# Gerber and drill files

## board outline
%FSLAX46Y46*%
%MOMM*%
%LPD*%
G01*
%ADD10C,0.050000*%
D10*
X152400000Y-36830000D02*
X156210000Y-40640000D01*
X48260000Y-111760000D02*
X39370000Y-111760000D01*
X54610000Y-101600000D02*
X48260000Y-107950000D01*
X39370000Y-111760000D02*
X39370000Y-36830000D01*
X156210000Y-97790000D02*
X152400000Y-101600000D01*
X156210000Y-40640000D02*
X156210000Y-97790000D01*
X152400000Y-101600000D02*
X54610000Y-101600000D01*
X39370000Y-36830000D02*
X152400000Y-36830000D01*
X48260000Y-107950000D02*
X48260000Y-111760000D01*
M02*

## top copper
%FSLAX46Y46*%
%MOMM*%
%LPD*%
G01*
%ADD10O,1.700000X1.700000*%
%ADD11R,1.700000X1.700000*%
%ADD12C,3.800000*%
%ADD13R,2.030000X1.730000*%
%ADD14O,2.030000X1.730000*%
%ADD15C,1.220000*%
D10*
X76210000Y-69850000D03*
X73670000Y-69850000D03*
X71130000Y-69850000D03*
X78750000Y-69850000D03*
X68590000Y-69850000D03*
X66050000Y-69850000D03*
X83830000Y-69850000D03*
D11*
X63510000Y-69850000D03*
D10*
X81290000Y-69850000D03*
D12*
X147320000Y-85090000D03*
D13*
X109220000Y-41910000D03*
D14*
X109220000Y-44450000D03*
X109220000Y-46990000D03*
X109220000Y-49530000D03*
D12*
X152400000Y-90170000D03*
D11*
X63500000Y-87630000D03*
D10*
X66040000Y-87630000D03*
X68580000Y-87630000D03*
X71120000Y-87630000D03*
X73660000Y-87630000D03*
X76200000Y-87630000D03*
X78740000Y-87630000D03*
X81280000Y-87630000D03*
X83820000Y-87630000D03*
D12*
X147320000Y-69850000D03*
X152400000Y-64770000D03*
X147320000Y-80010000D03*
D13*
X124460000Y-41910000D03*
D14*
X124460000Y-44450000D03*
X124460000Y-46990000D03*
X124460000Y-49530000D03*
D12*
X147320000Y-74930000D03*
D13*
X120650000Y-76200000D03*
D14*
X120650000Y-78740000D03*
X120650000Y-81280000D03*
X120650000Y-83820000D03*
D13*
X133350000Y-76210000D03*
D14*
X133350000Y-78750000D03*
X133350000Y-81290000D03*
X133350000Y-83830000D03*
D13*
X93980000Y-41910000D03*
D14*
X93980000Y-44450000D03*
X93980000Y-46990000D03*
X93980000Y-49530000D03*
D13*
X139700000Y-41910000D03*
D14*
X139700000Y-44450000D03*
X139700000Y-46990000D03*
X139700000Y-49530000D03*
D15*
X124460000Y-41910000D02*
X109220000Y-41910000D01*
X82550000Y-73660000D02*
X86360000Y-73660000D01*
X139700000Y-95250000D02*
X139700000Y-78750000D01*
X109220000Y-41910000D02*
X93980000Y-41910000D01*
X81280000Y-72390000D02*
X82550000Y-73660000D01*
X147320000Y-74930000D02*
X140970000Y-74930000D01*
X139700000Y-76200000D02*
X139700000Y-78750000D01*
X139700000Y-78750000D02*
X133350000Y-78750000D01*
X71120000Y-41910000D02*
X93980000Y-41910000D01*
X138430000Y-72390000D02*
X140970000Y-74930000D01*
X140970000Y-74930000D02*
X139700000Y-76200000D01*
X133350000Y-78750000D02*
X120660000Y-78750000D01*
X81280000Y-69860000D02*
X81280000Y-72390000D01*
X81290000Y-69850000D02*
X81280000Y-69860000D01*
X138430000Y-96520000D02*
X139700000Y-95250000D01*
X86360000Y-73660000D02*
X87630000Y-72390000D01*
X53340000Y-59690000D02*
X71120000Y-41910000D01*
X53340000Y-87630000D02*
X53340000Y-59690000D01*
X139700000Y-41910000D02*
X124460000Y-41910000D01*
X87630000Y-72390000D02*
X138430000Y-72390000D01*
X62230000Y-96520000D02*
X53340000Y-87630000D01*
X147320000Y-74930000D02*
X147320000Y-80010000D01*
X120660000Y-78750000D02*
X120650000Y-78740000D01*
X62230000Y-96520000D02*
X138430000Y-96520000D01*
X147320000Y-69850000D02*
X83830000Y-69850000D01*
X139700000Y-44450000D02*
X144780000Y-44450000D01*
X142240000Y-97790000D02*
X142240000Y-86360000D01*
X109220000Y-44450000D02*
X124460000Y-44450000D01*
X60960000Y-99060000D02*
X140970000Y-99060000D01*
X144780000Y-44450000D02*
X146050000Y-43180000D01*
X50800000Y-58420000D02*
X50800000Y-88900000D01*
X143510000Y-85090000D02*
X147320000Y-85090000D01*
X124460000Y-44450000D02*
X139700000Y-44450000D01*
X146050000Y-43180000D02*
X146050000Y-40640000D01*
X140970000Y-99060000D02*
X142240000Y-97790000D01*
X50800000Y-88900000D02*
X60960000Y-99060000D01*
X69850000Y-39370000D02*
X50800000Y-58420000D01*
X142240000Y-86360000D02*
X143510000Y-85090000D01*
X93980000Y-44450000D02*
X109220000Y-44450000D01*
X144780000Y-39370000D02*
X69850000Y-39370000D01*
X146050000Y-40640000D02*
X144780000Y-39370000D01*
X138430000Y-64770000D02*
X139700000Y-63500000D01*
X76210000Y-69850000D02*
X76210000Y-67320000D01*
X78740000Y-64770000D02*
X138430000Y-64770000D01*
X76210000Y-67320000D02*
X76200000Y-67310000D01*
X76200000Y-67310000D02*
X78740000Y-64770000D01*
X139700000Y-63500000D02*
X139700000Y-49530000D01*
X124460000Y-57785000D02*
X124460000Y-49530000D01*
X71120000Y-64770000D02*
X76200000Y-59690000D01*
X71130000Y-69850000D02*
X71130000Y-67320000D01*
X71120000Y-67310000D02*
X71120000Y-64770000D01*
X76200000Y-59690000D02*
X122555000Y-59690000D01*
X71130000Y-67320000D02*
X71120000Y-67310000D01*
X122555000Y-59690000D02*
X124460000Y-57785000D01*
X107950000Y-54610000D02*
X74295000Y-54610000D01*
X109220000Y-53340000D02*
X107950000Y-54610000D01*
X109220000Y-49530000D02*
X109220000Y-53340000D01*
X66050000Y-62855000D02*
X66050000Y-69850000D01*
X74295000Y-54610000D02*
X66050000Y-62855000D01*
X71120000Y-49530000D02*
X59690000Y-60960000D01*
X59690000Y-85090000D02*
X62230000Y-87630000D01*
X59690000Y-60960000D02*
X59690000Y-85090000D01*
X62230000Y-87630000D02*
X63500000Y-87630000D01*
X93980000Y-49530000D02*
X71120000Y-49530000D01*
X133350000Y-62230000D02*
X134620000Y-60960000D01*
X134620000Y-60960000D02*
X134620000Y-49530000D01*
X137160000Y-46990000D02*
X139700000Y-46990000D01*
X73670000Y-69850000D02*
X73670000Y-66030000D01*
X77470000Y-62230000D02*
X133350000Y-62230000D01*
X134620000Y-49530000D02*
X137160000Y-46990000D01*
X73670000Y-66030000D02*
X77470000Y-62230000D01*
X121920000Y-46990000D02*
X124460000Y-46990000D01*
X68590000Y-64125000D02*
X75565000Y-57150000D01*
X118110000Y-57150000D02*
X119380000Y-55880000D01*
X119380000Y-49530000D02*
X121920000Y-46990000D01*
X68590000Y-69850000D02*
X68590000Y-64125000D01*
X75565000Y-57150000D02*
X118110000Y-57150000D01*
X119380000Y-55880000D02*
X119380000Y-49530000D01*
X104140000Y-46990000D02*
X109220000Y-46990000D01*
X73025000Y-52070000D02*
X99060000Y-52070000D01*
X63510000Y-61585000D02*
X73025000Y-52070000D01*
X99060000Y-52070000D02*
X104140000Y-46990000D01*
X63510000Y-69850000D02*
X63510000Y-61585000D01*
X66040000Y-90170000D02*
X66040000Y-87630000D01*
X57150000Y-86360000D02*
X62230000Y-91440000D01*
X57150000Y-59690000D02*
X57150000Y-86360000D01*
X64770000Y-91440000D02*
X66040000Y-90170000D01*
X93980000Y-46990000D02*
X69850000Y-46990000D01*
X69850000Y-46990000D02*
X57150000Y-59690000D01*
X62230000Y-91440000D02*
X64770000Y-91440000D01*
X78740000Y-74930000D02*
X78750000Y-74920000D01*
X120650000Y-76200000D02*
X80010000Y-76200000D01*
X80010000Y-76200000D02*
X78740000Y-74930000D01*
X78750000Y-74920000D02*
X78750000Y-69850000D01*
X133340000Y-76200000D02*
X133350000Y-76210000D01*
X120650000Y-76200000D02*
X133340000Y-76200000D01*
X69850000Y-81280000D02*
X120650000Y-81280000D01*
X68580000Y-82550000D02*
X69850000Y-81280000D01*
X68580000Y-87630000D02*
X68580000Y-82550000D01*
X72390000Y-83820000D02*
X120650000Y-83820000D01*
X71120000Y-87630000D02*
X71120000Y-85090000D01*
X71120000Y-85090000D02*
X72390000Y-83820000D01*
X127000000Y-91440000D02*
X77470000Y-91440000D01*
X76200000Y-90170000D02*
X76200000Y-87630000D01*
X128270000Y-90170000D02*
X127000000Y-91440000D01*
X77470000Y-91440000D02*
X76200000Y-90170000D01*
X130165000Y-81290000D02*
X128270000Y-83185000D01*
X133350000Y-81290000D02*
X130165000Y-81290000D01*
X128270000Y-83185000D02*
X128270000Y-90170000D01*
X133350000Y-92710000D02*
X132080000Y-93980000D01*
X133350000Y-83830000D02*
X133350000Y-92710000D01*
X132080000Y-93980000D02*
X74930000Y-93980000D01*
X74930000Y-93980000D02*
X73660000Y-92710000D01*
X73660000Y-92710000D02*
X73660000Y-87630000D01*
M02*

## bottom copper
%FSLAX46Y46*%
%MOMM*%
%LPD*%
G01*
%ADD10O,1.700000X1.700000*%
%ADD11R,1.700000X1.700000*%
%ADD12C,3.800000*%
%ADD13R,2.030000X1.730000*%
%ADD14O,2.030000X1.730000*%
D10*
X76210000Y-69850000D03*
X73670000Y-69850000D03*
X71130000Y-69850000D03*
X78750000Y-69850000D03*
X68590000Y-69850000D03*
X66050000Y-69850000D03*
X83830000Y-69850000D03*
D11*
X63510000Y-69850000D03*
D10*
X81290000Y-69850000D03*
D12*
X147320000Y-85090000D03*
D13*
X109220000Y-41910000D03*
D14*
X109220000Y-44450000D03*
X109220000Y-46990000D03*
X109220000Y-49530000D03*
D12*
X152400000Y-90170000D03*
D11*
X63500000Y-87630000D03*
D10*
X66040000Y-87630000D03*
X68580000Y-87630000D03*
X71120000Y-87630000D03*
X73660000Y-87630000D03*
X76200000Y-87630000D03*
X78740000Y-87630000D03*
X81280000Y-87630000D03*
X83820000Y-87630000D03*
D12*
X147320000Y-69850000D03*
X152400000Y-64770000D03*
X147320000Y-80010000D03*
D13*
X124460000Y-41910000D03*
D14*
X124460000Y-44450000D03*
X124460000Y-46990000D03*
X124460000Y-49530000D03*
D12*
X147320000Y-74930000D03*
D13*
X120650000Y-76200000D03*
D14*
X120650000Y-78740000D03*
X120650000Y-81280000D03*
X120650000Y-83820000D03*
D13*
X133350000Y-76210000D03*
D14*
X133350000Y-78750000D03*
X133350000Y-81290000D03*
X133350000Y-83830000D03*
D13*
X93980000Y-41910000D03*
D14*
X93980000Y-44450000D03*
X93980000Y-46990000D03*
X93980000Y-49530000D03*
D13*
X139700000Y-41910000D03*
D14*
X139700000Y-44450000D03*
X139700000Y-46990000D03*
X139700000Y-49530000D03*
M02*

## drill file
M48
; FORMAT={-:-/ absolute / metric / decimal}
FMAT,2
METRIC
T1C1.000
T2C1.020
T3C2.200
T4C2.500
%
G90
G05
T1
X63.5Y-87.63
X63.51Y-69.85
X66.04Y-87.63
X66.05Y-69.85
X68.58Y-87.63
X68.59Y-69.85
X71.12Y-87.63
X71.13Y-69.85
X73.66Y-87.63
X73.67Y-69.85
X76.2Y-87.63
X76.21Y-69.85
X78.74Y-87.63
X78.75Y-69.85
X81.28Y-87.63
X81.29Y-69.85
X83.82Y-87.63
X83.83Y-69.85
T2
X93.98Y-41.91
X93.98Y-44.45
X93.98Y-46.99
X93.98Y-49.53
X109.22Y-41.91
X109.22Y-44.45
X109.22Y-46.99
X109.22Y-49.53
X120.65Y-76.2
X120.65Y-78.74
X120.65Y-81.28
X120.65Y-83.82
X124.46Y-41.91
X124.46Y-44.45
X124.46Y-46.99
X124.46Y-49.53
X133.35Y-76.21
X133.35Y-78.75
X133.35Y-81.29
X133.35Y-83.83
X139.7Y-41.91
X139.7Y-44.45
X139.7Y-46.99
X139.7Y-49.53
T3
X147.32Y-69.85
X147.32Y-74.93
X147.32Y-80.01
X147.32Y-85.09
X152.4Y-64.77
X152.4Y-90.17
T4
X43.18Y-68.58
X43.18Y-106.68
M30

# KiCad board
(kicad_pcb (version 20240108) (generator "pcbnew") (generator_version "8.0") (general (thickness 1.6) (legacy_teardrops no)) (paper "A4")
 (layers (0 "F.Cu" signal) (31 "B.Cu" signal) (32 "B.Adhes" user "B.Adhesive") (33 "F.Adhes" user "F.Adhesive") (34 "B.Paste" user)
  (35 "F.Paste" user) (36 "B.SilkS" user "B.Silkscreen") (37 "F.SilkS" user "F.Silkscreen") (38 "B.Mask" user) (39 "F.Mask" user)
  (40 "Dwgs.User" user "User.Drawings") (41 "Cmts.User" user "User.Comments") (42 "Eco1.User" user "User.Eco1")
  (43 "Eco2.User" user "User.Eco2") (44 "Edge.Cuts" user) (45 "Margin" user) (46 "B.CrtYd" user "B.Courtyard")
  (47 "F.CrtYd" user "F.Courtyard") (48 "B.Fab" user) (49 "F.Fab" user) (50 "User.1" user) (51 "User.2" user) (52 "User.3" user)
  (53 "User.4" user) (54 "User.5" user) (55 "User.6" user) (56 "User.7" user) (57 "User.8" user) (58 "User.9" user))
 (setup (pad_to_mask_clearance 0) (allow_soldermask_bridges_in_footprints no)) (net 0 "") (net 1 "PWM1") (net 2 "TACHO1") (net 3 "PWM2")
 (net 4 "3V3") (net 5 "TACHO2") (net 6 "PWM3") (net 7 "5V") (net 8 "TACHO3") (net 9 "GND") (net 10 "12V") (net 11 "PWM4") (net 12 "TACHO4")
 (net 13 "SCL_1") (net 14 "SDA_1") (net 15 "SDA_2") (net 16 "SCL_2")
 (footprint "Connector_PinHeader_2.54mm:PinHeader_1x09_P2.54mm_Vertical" (layer "F.Cu") (at 63.51 69.85 90)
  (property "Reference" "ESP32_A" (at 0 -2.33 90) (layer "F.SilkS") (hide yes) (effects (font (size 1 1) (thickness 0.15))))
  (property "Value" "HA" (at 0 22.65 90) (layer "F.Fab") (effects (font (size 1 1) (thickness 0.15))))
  (pad "1" thru_hole oval (at 0 12.7 90) (size 1.7 1.7) (drill 1) (layers "*.Cu" "*.Mask") (remove_unused_layers no) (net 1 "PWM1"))
  (pad "2" thru_hole oval (at 0 10.16 90) (size 1.7 1.7) (drill 1) (layers "*.Cu" "*.Mask") (remove_unused_layers no) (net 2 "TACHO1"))
  (pad "3" thru_hole oval (at 0 7.62 90) (size 1.7 1.7) (drill 1) (layers "*.Cu" "*.Mask") (remove_unused_layers no) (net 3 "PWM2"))
  (pad "3V3" thru_hole oval (at 0 15.24 90) (size 1.7 1.7) (drill 1) (layers "*.Cu" "*.Mask") (remove_unused_layers no) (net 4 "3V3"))
  (pad "4" thru_hole oval (at 0 5.08 90) (size 1.7 1.7) (drill 1) (layers "*.Cu" "*.Mask") (remove_unused_layers no) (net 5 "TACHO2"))
  (pad "5" thru_hole oval (at 0 2.54 90) (size 1.7 1.7) (drill 1) (layers "*.Cu" "*.Mask") (remove_unused_layers no) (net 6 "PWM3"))
  (pad "5V" thru_hole oval (at 0 20.32 90) (size 1.7 1.7) (drill 1) (layers "*.Cu" "*.Mask") (remove_unused_layers no) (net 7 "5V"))
  (pad "6" thru_hole rect (at 0 0 90) (size 1.7 1.7) (drill 1) (layers "*.Cu" "*.Mask") (remove_unused_layers no) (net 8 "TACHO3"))
  (pad "GND" thru_hole oval (at 0 17.78 90) (size 1.7 1.7) (drill 1) (layers "*.Cu" "*.Mask") (remove_unused_layers no) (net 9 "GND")))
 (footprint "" (layer "F.Cu") (at 147.32 85.09)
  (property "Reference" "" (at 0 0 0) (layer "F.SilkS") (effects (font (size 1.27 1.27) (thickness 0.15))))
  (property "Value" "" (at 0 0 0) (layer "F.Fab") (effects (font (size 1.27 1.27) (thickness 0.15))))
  (pad "1" thru_hole circle (at 0 0) (size 3.8 3.8) (drill 2.2) (layers "*.Cu" "*.Mask") (remove_unused_layers no) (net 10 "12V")))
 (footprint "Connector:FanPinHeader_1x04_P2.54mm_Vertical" (layer "F.Cu") (at 109.22 41.91 -90)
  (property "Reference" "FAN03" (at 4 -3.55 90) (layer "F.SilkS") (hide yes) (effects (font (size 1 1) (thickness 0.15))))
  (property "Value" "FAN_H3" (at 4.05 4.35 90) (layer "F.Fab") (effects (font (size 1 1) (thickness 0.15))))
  (pad "1" thru_hole rect (at 0 0) (size 2.03 1.73) (drill 1.02) (layers "*.Cu" "*.Mask") (remove_unused_layers no) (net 9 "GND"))
  (pad "2" thru_hole oval (at 2.54 0) (size 2.03 1.73) (drill 1.02) (layers "*.Cu" "*.Mask") (remove_unused_layers no) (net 10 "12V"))
  (pad "3" thru_hole oval (at 5.08 0) (size 2.03 1.73) (drill 1.02) (layers "*.Cu" "*.Mask") (remove_unused_layers no) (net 8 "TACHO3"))
  (pad "4" thru_hole oval (at 7.62 0) (size 2.03 1.73) (drill 1.02) (layers "*.Cu" "*.Mask") (remove_unused_layers no) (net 6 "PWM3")))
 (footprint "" (layer "F.Cu") (at 152.4 90.17)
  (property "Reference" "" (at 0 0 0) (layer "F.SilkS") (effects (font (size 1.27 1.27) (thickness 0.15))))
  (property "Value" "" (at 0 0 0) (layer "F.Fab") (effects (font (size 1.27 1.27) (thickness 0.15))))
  (pad "MNT" thru_hole circle (at 0 0) (size 3.8 3.8) (drill 2.2) (layers "*.Cu" "*.Mask") (remove_unused_layers no)))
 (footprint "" (layer "F.Cu") (at 43.18 106.68)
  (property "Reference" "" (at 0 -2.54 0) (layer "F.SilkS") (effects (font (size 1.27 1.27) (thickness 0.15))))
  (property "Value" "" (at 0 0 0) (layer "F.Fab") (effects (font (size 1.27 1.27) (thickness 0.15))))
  (pad "" np_thru_hole circle (at 0 0) (size 2.5 2.5) (drill 2.5) (layers "*.Cu" "*.Mask")))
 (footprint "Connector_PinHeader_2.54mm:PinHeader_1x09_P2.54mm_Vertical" (layer "F.Cu") (at 63.5 87.63 90)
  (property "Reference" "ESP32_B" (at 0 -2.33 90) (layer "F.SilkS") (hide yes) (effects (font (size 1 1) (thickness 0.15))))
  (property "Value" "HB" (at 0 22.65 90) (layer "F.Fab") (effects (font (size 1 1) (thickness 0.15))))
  (pad "7" thru_hole rect (at 0 0 90) (size 1.7 1.7) (drill 1) (layers "*.Cu" "*.Mask") (remove_unused_layers no) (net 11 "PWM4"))
  (pad "8" thru_hole oval (at 0 2.54 90) (size 1.7 1.7) (drill 1) (layers "*.Cu" "*.Mask") (remove_unused_layers no) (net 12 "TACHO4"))
  (pad "9" thru_hole oval (at 0 5.08 90) (size 1.7 1.7) (drill 1) (layers "*.Cu" "*.Mask") (remove_unused_layers no) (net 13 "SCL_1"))
  (pad "10" thru_hole oval (at 0 7.62 90) (size 1.7 1.7) (drill 1) (layers "*.Cu" "*.Mask") (remove_unused_layers no) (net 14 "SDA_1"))
  (pad "11" thru_hole oval (at 0 10.16 90) (size 1.7 1.7) (drill 1) (layers "*.Cu" "*.Mask") (remove_unused_layers no) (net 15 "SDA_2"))
  (pad "12" thru_hole oval (at 0 12.7 90) (size 1.7 1.7) (drill 1) (layers "*.Cu" "*.Mask") (remove_unused_layers no) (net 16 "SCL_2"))
  (pad "13" thru_hole oval (at 0 15.24 90) (size 1.7 1.7) (drill 1) (layers "*.Cu" "*.Mask") (remove_unused_layers no))
  (pad "RX" thru_hole oval (at 0 17.78 90) (size 1.7 1.7) (drill 1) (layers "*.Cu" "*.Mask") (remove_unused_layers no))
  (pad "TX" thru_hole oval (at 0 20.32 90) (size 1.7 1.7) (drill 1) (layers "*.Cu" "*.Mask") (remove_unused_layers no)))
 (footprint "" (layer "F.Cu") (at 147.32 69.85)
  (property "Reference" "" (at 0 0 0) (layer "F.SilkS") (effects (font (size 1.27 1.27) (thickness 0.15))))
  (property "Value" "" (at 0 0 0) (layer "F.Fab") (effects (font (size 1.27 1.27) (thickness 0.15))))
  (pad "4" thru_hole circle (at 0 0) (size 3.8 3.8) (drill 2.2) (layers "*.Cu" "*.Mask") (remove_unused_layers no) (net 7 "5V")))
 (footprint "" (layer "F.Cu") (at 152.4 64.77)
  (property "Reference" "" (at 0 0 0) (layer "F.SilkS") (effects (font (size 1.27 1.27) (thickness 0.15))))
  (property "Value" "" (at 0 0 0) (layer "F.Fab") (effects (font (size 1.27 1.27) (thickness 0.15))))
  (pad "MNT" thru_hole circle (at 0 0) (size 3.8 3.8) (drill 2.2) (layers "*.Cu" "*.Mask") (remove_unused_layers no)))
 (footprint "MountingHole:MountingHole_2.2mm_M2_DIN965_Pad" (layer "F.Cu") (at 147.32 80.01)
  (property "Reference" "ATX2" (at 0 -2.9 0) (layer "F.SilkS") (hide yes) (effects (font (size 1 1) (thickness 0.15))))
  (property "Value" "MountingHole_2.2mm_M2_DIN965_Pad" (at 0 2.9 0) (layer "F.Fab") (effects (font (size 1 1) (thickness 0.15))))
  (pad "2" thru_hole circle (at 0 0) (size 3.8 3.8) (drill 2.2) (layers "*.Cu" "*.Mask") (remove_unused_layers no) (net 9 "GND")))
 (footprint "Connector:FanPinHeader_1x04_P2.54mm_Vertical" (layer "F.Cu") (at 124.46 41.91 -90)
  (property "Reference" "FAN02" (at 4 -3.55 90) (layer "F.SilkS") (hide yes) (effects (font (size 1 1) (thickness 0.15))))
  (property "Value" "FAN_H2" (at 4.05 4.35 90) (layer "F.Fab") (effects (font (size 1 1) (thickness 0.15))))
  (pad "1" thru_hole rect (at 0 0) (size 2.03 1.73) (drill 1.02) (layers "*.Cu" "*.Mask") (remove_unused_layers no) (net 9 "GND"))
  (pad "2" thru_hole oval (at 2.54 0) (size 2.03 1.73) (drill 1.02) (layers "*.Cu" "*.Mask") (remove_unused_layers no) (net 10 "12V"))
  (pad "3" thru_hole oval (at 5.08 0) (size 2.03 1.73) (drill 1.02) (layers "*.Cu" "*.Mask") (remove_unused_layers no) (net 5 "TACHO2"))
  (pad "4" thru_hole oval (at 7.62 0) (size 2.03 1.73) (drill 1.02) (layers "*.Cu" "*.Mask") (remove_unused_layers no) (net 3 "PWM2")))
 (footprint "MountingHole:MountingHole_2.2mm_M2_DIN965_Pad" (layer "F.Cu") (at 147.32 74.93)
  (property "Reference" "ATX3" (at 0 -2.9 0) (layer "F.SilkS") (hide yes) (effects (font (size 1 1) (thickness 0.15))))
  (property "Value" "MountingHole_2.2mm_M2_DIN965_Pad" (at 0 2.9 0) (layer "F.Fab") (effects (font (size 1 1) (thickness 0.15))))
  (pad "3" thru_hole circle (at 0 0) (size 3.8 3.8) (drill 2.2) (layers "*.Cu" "*.Mask") (remove_unused_layers no) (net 9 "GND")))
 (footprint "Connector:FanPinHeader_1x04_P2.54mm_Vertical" (layer "F.Cu") (at 120.65 76.2 -90)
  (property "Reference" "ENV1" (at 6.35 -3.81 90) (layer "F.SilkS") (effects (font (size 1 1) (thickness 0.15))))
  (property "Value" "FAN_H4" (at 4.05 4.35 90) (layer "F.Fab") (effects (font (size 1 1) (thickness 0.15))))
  (pad "1" thru_hole rect (at 0 0) (size 2.03 1.73) (drill 1.02) (layers "*.Cu" "*.Mask") (remove_unused_layers no) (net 4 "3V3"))
  (pad "2" thru_hole oval (at 2.54 0) (size 2.03 1.73) (drill 1.02) (layers "*.Cu" "*.Mask") (remove_unused_layers no) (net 9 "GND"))
  (pad "3" thru_hole oval (at 5.08 0) (size 2.03 1.73) (drill 1.02) (layers "*.Cu" "*.Mask") (remove_unused_layers no) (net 13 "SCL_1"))
  (pad "4" thru_hole oval (at 7.62 0) (size 2.03 1.73) (drill 1.02) (layers "*.Cu" "*.Mask") (remove_unused_layers no) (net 14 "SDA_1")))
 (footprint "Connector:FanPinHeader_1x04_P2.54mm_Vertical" (layer "F.Cu") (at 133.35 76.21 -90)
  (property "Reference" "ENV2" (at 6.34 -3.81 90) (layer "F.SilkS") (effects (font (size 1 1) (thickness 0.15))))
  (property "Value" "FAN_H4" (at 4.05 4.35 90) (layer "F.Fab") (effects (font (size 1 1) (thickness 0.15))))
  (pad "1" thru_hole rect (at 0 0) (size 2.03 1.73) (drill 1.02) (layers "*.Cu" "*.Mask") (remove_unused_layers no) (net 4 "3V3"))
  (pad "2" thru_hole oval (at 2.54 0) (size 2.03 1.73) (drill 1.02) (layers "*.Cu" "*.Mask") (remove_unused_layers no) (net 9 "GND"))
  (pad "3" thru_hole oval (at 5.08 0) (size 2.03 1.73) (drill 1.02) (layers "*.Cu" "*.Mask") (remove_unused_layers no) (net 16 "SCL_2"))
  (pad "4" thru_hole oval (at 7.62 0) (size 2.03 1.73) (drill 1.02) (layers "*.Cu" "*.Mask") (remove_unused_layers no) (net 15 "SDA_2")))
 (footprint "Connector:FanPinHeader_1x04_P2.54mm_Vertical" (layer "F.Cu") (at 93.98 41.91 -90)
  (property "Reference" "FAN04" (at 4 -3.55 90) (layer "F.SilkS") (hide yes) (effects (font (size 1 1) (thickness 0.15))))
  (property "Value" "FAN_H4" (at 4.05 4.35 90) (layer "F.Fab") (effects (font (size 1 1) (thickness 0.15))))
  (pad "1" thru_hole rect (at 0 0) (size 2.03 1.73) (drill 1.02) (layers "*.Cu" "*.Mask") (remove_unused_layers no) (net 9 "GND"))
  (pad "2" thru_hole oval (at 2.54 0) (size 2.03 1.73) (drill 1.02) (layers "*.Cu" "*.Mask") (remove_unused_layers no) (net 10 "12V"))
  (pad "3" thru_hole oval (at 5.08 0) (size 2.03 1.73) (drill 1.02) (layers "*.Cu" "*.Mask") (remove_unused_layers no) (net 12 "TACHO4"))
  (pad "4" thru_hole oval (at 7.62 0) (size 2.03 1.73) (drill 1.02) (layers "*.Cu" "*.Mask") (remove_unused_layers no) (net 11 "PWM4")))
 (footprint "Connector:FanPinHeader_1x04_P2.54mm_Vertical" (layer "F.Cu") (at 139.7 41.91 -90)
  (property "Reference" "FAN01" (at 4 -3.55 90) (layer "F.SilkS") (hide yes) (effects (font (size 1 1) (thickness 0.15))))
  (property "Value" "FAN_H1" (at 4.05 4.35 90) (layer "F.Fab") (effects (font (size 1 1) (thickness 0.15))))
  (pad "1" thru_hole rect (at 0 0) (size 2.03 1.73) (drill 1.02) (layers "*.Cu" "*.Mask") (remove_unused_layers no) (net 9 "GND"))
  (pad "2" thru_hole oval (at 2.54 0) (size 2.03 1.73) (drill 1.02) (layers "*.Cu" "*.Mask") (remove_unused_layers no) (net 10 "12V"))
  (pad "3" thru_hole oval (at 5.08 0) (size 2.03 1.73) (drill 1.02) (layers "*.Cu" "*.Mask") (remove_unused_layers no) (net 2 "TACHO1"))
  (pad "4" thru_hole oval (at 7.62 0) (size 2.03 1.73) (drill 1.02) (layers "*.Cu" "*.Mask") (remove_unused_layers no) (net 1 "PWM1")))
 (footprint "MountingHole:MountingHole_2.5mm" (layer "F.Cu") (at 43.18 68.58)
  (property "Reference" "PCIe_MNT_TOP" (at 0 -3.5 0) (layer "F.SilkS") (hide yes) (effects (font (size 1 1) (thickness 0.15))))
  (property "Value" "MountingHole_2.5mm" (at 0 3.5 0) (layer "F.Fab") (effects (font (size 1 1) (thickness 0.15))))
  (pad "" np_thru_hole circle (at 0 0) (size 2.5 2.5) (drill 2.5) (layers "*.Cu" "*.Mask")))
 (gr_line (start 152.4 36.83) (end 156.21 40.64) (stroke (width 0.05) (type default)) (layer "Edge.Cuts"))
 (gr_line (start 48.26 111.76) (end 39.37 111.76) (stroke (width 0.05) (type default)) (layer "Edge.Cuts"))
 (gr_line (start 54.61 101.6) (end 48.26 107.95) (stroke (width 0.05) (type default)) (layer "Edge.Cuts"))
 (gr_line (start 39.37 111.76) (end 39.37 36.83) (stroke (width 0.05) (type default)) (layer "Edge.Cuts"))
 (gr_line (start 156.21 97.79) (end 152.4 101.6) (stroke (width 0.05) (type default)) (layer "Edge.Cuts"))
 (gr_line (start 156.21 40.64) (end 156.21 97.79) (stroke (width 0.05) (type default)) (layer "Edge.Cuts"))
 (gr_line (start 152.4 101.6) (end 54.61 101.6) (stroke (width 0.05) (type default)) (layer "Edge.Cuts"))
 (gr_line (start 39.37 36.83) (end 152.4 36.83) (stroke (width 0.05) (type default)) (layer "Edge.Cuts"))
 (gr_line (start 48.26 107.95) (end 48.26 111.76) (stroke (width 0.05) (type default)) (layer "Edge.Cuts"))
 (segment (start 124.46 41.91) (end 109.22 41.91) (width 1.22) (layer "F.Cu") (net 9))
 (segment (start 82.55 73.66) (end 86.36 73.66) (width 1.22) (layer "F.Cu") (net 9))
 (segment (start 139.7 95.25) (end 139.7 78.75) (width 1.22) (layer "F.Cu") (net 9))
 (segment (start 109.22 41.91) (end 93.98 41.91) (width 1.22) (layer "F.Cu") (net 9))
 (segment (start 81.28 72.39) (end 82.55 73.66) (width 1.22) (layer "F.Cu") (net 9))
 (segment (start 147.32 74.93) (end 140.97 74.93) (width 1.22) (layer "F.Cu") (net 9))
 (segment (start 139.7 76.2) (end 139.7 78.75) (width 1.22) (layer "F.Cu") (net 9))
 (segment (start 139.7 78.75) (end 133.35 78.75) (width 1.22) (layer "F.Cu") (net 9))
 (segment (start 71.12 41.91) (end 93.98 41.91) (width 1.22) (layer "F.Cu") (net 9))
 (segment (start 138.43 72.39) (end 140.97 74.93) (width 1.22) (layer "F.Cu") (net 9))
 (segment (start 140.97 74.93) (end 139.7 76.2) (width 1.22) (layer "F.Cu") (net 9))
 (segment (start 133.35 78.75) (end 120.66 78.75) (width 1.22) (layer "F.Cu") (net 9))
 (segment (start 81.28 69.86) (end 81.28 72.39) (width 1.22) (layer "F.Cu") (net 9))
 (segment (start 81.29 69.85) (end 81.28 69.86) (width 1.22) (layer "F.Cu") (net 9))
 (segment (start 138.43 96.52) (end 139.7 95.25) (width 1.22) (layer "F.Cu") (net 9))
 (segment (start 86.36 73.66) (end 87.63 72.39) (width 1.22) (layer "F.Cu") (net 9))
 (segment (start 53.34 59.69) (end 71.12 41.91) (width 1.22) (layer "F.Cu") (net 9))
 (segment (start 53.34 87.63) (end 53.34 59.69) (width 1.22) (layer "F.Cu") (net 9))
 (segment (start 139.7 41.91) (end 124.46 41.91) (width 1.22) (layer "F.Cu") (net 9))
 (segment (start 87.63 72.39) (end 138.43 72.39) (width 1.22) (layer "F.Cu") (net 9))
 (segment (start 62.23 96.52) (end 53.34 87.63) (width 1.22) (layer "F.Cu") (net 9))
 (segment (start 147.32 74.93) (end 147.32 80.01) (width 1.22) (layer "F.Cu") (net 9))
 (segment (start 120.66 78.75) (end 120.65 78.74) (width 1.22) (layer "F.Cu") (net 9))
 (segment (start 62.23 96.52) (end 138.43 96.52) (width 1.22) (layer "F.Cu") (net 9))
 (segment (start 147.32 69.85) (end 83.83 69.85) (width 1.22) (layer "F.Cu") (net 7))
 (segment (start 139.7 44.45) (end 144.78 44.45) (width 1.22) (layer "F.Cu") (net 10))
 (segment (start 142.24 97.79) (end 142.24 86.36) (width 1.22) (layer "F.Cu") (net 10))
 (segment (start 109.22 44.45) (end 124.46 44.45) (width 1.22) (layer "F.Cu") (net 10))
 (segment (start 60.96 99.06) (end 140.97 99.06) (width 1.22) (layer "F.Cu") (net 10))
 (segment (start 144.78 44.45) (end 146.05 43.18) (width 1.22) (layer "F.Cu") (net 10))
 (segment (start 50.8 58.42) (end 50.8 88.9) (width 1.22) (layer "F.Cu") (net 10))
 (segment (start 143.51 85.09) (end 147.32 85.09) (width 1.22) (layer "F.Cu") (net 10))
 (segment (start 124.46 44.45) (end 139.7 44.45) (width 1.22) (layer "F.Cu") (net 10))
 (segment (start 146.05 43.18) (end 146.05 40.64) (width 1.22) (layer "F.Cu") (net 10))
 (segment (start 140.97 99.06) (end 142.24 97.79) (width 1.22) (layer "F.Cu") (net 10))
 (segment (start 50.8 88.9) (end 60.96 99.06) (width 1.22) (layer "F.Cu") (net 10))
 (segment (start 69.85 39.37) (end 50.8 58.42) (width 1.22) (layer "F.Cu") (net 10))
 (segment (start 142.24 86.36) (end 143.51 85.09) (width 1.22) (layer "F.Cu") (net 10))
 (segment (start 93.98 44.45) (end 109.22 44.45) (width 1.22) (layer "F.Cu") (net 10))
 (segment (start 144.78 39.37) (end 69.85 39.37) (width 1.22) (layer "F.Cu") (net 10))
 (segment (start 146.05 40.64) (end 144.78 39.37) (width 1.22) (layer "F.Cu") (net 10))
 (segment (start 138.43 64.77) (end 139.7 63.5) (width 1.22) (layer "F.Cu") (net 1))
 (segment (start 76.21 69.85) (end 76.21 67.32) (width 1.22) (layer "F.Cu") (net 1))
 (segment (start 78.74 64.77) (end 138.43 64.77) (width 1.22) (layer "F.Cu") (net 1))
 (segment (start 76.21 67.32) (end 76.2 67.31) (width 1.22) (layer "F.Cu") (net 1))
 (segment (start 76.2 67.31) (end 78.74 64.77) (width 1.22) (layer "F.Cu") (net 1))
 (segment (start 139.7 63.5) (end 139.7 49.53) (width 1.22) (layer "F.Cu") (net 1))
 (segment (start 124.46 57.785) (end 124.46 49.53) (width 1.22) (layer "F.Cu") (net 3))
 (segment (start 71.12 64.77) (end 76.2 59.69) (width 1.22) (layer "F.Cu") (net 3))
 (segment (start 71.13 69.85) (end 71.13 67.32) (width 1.22) (layer "F.Cu") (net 3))
 (segment (start 71.12 67.31) (end 71.12 64.77) (width 1.22) (layer "F.Cu") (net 3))
 (segment (start 76.2 59.69) (end 122.555 59.69) (width 1.22) (layer "F.Cu") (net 3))
 (segment (start 71.13 67.32) (end 71.12 67.31) (width 1.22) (layer "F.Cu") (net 3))
 (segment (start 122.555 59.69) (end 124.46 57.785) (width 1.22) (layer "F.Cu") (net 3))
 (segment (start 107.95 54.61) (end 74.295 54.61) (width 1.22) (layer "F.Cu") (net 6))
 (segment (start 109.22 53.34) (end 107.95 54.61) (width 1.22) (layer "F.Cu") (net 6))
 (segment (start 109.22 49.53) (end 109.22 53.34) (width 1.22) (layer "F.Cu") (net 6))
 (segment (start 66.05 62.855) (end 66.05 69.85) (width 1.22) (layer "F.Cu") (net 6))
 (segment (start 74.295 54.61) (end 66.05 62.855) (width 1.22) (layer "F.Cu") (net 6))
 (segment (start 71.12 49.53) (end 59.69 60.96) (width 1.22) (layer "F.Cu") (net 11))
 (segment (start 59.69 85.09) (end 62.23 87.63) (width 1.22) (layer "F.Cu") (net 11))
 (segment (start 59.69 60.96) (end 59.69 85.09) (width 1.22) (layer "F.Cu") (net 11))
 (segment (start 62.23 87.63) (end 63.5 87.63) (width 1.22) (layer "F.Cu") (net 11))
 (segment (start 93.98 49.53) (end 71.12 49.53) (width 1.22) (layer "F.Cu") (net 11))
 (segment (start 133.35 62.23) (end 134.62 60.96) (width 1.22) (layer "F.Cu") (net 2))
 (segment (start 134.62 60.96) (end 134.62 49.53) (width 1.22) (layer "F.Cu") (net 2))
 (segment (start 137.16 46.99) (end 139.7 46.99) (width 1.22) (layer "F.Cu") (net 2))
 (segment (start 73.67 69.85) (end 73.67 66.03) (width 1.22) (layer "F.Cu") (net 2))
 (segment (start 77.47 62.23) (end 133.35 62.23) (width 1.22) (layer "F.Cu") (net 2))
 (segment (start 134.62 49.53) (end 137.16 46.99) (width 1.22) (layer "F.Cu") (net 2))
 (segment (start 73.67 66.03) (end 77.47 62.23) (width 1.22) (layer "F.Cu") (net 2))
 (segment (start 121.92 46.99) (end 124.46 46.99) (width 1.22) (layer "F.Cu") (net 5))
 (segment (start 68.59 64.125) (end 75.565 57.15) (width 1.22) (layer "F.Cu") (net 5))
 (segment (start 118.11 57.15) (end 119.38 55.88) (width 1.22) (layer "F.Cu") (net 5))
 (segment (start 119.38 49.53) (end 121.92 46.99) (width 1.22) (layer "F.Cu") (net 5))
 (segment (start 68.59 69.85) (end 68.59 64.125) (width 1.22) (layer "F.Cu") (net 5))
 (segment (start 75.565 57.15) (end 118.11 57.15) (width 1.22) (layer "F.Cu") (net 5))
 (segment (start 119.38 55.88) (end 119.38 49.53) (width 1.22) (layer "F.Cu") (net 5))
 (segment (start 104.14 46.99) (end 109.22 46.99) (width 1.22) (layer "F.Cu") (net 8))
 (segment (start 73.025 52.07) (end 99.06 52.07) (width 1.22) (layer "F.Cu") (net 8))
 (segment (start 63.51 61.585) (end 73.025 52.07) (width 1.22) (layer "F.Cu") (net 8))
 (segment (start 99.06 52.07) (end 104.14 46.99) (width 1.22) (layer "F.Cu") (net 8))
 (segment (start 63.51 69.85) (end 63.51 61.585) (width 1.22) (layer "F.Cu") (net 8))
 (segment (start 66.04 90.17) (end 66.04 87.63) (width 1.22) (layer "F.Cu") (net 12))
 (segment (start 57.15 86.36) (end 62.23 91.44) (width 1.22) (layer "F.Cu") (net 12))
 (segment (start 57.15 59.69) (end 57.15 86.36) (width 1.22) (layer "F.Cu") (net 12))
 (segment (start 64.77 91.44) (end 66.04 90.17) (width 1.22) (layer "F.Cu") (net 12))
 (segment (start 93.98 46.99) (end 69.85 46.99) (width 1.22) (layer "F.Cu") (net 12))
 (segment (start 69.85 46.99) (end 57.15 59.69) (width 1.22) (layer "F.Cu") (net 12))
 (segment (start 62.23 91.44) (end 64.77 91.44) (width 1.22) (layer "F.Cu") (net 12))
 (segment (start 78.74 74.93) (end 78.75 74.92) (width 1.22) (layer "F.Cu") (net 4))
 (segment (start 120.65 76.2) (end 80.01 76.2) (width 1.22) (layer "F.Cu") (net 4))
 (segment (start 80.01 76.2) (end 78.74 74.93) (width 1.22) (layer "F.Cu") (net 4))
 (segment (start 78.75 74.92) (end 78.75 69.85) (width 1.22) (layer "F.Cu") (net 4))
 (segment (start 133.34 76.2) (end 133.35 76.21) (width 1.22) (layer "F.Cu") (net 4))
 (segment (start 120.65 76.2) (end 133.34 76.2) (width 1.22) (layer "F.Cu") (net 4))
 (segment (start 69.85 81.28) (end 120.65 81.28) (width 1.22) (layer "F.Cu") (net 13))
 (segment (start 68.58 82.55) (end 69.85 81.28) (width 1.22) (layer "F.Cu") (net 13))
 (segment (start 68.58 87.63) (end 68.58 82.55) (width 1.22) (layer "F.Cu") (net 13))
 (segment (start 72.39 83.82) (end 120.65 83.82) (width 1.22) (layer "F.Cu") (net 14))
 (segment (start 71.12 87.63) (end 71.12 85.09) (width 1.22) (layer "F.Cu") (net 14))
 (segment (start 71.12 85.09) (end 72.39 83.82) (width 1.22) (layer "F.Cu") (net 14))
 (segment (start 127 91.44) (end 77.47 91.44) (width 1.22) (layer "F.Cu") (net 16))
 (segment (start 76.2 90.17) (end 76.2 87.63) (width 1.22) (layer "F.Cu") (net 16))
 (segment (start 128.27 90.17) (end 127 91.44) (width 1.22) (layer "F.Cu") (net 16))
 (segment (start 77.47 91.44) (end 76.2 90.17) (width 1.22) (layer "F.Cu") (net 16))
 (segment (start 130.165 81.29) (end 128.27 83.185) (width 1.22) (layer "F.Cu") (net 16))
 (segment (start 133.35 81.29) (end 130.165 81.29) (width 1.22) (layer "F.Cu") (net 16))
 (segment (start 128.27 83.185) (end 128.27 90.17) (width 1.22) (layer "F.Cu") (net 16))
 (segment (start 133.35 92.71) (end 132.08 93.98) (width 1.22) (layer "F.Cu") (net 15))
 (segment (start 133.35 83.83) (end 133.35 92.71) (width 1.22) (layer "F.Cu") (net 15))
 (segment (start 132.08 93.98) (end 74.93 93.98) (width 1.22) (layer "F.Cu") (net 15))
 (segment (start 74.93 93.98) (end 73.66 92.71) (width 1.22) (layer "F.Cu") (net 15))
 (segment (start 73.66 92.71) (end 73.66 87.63) (width 1.22) (layer "F.Cu") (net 15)))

